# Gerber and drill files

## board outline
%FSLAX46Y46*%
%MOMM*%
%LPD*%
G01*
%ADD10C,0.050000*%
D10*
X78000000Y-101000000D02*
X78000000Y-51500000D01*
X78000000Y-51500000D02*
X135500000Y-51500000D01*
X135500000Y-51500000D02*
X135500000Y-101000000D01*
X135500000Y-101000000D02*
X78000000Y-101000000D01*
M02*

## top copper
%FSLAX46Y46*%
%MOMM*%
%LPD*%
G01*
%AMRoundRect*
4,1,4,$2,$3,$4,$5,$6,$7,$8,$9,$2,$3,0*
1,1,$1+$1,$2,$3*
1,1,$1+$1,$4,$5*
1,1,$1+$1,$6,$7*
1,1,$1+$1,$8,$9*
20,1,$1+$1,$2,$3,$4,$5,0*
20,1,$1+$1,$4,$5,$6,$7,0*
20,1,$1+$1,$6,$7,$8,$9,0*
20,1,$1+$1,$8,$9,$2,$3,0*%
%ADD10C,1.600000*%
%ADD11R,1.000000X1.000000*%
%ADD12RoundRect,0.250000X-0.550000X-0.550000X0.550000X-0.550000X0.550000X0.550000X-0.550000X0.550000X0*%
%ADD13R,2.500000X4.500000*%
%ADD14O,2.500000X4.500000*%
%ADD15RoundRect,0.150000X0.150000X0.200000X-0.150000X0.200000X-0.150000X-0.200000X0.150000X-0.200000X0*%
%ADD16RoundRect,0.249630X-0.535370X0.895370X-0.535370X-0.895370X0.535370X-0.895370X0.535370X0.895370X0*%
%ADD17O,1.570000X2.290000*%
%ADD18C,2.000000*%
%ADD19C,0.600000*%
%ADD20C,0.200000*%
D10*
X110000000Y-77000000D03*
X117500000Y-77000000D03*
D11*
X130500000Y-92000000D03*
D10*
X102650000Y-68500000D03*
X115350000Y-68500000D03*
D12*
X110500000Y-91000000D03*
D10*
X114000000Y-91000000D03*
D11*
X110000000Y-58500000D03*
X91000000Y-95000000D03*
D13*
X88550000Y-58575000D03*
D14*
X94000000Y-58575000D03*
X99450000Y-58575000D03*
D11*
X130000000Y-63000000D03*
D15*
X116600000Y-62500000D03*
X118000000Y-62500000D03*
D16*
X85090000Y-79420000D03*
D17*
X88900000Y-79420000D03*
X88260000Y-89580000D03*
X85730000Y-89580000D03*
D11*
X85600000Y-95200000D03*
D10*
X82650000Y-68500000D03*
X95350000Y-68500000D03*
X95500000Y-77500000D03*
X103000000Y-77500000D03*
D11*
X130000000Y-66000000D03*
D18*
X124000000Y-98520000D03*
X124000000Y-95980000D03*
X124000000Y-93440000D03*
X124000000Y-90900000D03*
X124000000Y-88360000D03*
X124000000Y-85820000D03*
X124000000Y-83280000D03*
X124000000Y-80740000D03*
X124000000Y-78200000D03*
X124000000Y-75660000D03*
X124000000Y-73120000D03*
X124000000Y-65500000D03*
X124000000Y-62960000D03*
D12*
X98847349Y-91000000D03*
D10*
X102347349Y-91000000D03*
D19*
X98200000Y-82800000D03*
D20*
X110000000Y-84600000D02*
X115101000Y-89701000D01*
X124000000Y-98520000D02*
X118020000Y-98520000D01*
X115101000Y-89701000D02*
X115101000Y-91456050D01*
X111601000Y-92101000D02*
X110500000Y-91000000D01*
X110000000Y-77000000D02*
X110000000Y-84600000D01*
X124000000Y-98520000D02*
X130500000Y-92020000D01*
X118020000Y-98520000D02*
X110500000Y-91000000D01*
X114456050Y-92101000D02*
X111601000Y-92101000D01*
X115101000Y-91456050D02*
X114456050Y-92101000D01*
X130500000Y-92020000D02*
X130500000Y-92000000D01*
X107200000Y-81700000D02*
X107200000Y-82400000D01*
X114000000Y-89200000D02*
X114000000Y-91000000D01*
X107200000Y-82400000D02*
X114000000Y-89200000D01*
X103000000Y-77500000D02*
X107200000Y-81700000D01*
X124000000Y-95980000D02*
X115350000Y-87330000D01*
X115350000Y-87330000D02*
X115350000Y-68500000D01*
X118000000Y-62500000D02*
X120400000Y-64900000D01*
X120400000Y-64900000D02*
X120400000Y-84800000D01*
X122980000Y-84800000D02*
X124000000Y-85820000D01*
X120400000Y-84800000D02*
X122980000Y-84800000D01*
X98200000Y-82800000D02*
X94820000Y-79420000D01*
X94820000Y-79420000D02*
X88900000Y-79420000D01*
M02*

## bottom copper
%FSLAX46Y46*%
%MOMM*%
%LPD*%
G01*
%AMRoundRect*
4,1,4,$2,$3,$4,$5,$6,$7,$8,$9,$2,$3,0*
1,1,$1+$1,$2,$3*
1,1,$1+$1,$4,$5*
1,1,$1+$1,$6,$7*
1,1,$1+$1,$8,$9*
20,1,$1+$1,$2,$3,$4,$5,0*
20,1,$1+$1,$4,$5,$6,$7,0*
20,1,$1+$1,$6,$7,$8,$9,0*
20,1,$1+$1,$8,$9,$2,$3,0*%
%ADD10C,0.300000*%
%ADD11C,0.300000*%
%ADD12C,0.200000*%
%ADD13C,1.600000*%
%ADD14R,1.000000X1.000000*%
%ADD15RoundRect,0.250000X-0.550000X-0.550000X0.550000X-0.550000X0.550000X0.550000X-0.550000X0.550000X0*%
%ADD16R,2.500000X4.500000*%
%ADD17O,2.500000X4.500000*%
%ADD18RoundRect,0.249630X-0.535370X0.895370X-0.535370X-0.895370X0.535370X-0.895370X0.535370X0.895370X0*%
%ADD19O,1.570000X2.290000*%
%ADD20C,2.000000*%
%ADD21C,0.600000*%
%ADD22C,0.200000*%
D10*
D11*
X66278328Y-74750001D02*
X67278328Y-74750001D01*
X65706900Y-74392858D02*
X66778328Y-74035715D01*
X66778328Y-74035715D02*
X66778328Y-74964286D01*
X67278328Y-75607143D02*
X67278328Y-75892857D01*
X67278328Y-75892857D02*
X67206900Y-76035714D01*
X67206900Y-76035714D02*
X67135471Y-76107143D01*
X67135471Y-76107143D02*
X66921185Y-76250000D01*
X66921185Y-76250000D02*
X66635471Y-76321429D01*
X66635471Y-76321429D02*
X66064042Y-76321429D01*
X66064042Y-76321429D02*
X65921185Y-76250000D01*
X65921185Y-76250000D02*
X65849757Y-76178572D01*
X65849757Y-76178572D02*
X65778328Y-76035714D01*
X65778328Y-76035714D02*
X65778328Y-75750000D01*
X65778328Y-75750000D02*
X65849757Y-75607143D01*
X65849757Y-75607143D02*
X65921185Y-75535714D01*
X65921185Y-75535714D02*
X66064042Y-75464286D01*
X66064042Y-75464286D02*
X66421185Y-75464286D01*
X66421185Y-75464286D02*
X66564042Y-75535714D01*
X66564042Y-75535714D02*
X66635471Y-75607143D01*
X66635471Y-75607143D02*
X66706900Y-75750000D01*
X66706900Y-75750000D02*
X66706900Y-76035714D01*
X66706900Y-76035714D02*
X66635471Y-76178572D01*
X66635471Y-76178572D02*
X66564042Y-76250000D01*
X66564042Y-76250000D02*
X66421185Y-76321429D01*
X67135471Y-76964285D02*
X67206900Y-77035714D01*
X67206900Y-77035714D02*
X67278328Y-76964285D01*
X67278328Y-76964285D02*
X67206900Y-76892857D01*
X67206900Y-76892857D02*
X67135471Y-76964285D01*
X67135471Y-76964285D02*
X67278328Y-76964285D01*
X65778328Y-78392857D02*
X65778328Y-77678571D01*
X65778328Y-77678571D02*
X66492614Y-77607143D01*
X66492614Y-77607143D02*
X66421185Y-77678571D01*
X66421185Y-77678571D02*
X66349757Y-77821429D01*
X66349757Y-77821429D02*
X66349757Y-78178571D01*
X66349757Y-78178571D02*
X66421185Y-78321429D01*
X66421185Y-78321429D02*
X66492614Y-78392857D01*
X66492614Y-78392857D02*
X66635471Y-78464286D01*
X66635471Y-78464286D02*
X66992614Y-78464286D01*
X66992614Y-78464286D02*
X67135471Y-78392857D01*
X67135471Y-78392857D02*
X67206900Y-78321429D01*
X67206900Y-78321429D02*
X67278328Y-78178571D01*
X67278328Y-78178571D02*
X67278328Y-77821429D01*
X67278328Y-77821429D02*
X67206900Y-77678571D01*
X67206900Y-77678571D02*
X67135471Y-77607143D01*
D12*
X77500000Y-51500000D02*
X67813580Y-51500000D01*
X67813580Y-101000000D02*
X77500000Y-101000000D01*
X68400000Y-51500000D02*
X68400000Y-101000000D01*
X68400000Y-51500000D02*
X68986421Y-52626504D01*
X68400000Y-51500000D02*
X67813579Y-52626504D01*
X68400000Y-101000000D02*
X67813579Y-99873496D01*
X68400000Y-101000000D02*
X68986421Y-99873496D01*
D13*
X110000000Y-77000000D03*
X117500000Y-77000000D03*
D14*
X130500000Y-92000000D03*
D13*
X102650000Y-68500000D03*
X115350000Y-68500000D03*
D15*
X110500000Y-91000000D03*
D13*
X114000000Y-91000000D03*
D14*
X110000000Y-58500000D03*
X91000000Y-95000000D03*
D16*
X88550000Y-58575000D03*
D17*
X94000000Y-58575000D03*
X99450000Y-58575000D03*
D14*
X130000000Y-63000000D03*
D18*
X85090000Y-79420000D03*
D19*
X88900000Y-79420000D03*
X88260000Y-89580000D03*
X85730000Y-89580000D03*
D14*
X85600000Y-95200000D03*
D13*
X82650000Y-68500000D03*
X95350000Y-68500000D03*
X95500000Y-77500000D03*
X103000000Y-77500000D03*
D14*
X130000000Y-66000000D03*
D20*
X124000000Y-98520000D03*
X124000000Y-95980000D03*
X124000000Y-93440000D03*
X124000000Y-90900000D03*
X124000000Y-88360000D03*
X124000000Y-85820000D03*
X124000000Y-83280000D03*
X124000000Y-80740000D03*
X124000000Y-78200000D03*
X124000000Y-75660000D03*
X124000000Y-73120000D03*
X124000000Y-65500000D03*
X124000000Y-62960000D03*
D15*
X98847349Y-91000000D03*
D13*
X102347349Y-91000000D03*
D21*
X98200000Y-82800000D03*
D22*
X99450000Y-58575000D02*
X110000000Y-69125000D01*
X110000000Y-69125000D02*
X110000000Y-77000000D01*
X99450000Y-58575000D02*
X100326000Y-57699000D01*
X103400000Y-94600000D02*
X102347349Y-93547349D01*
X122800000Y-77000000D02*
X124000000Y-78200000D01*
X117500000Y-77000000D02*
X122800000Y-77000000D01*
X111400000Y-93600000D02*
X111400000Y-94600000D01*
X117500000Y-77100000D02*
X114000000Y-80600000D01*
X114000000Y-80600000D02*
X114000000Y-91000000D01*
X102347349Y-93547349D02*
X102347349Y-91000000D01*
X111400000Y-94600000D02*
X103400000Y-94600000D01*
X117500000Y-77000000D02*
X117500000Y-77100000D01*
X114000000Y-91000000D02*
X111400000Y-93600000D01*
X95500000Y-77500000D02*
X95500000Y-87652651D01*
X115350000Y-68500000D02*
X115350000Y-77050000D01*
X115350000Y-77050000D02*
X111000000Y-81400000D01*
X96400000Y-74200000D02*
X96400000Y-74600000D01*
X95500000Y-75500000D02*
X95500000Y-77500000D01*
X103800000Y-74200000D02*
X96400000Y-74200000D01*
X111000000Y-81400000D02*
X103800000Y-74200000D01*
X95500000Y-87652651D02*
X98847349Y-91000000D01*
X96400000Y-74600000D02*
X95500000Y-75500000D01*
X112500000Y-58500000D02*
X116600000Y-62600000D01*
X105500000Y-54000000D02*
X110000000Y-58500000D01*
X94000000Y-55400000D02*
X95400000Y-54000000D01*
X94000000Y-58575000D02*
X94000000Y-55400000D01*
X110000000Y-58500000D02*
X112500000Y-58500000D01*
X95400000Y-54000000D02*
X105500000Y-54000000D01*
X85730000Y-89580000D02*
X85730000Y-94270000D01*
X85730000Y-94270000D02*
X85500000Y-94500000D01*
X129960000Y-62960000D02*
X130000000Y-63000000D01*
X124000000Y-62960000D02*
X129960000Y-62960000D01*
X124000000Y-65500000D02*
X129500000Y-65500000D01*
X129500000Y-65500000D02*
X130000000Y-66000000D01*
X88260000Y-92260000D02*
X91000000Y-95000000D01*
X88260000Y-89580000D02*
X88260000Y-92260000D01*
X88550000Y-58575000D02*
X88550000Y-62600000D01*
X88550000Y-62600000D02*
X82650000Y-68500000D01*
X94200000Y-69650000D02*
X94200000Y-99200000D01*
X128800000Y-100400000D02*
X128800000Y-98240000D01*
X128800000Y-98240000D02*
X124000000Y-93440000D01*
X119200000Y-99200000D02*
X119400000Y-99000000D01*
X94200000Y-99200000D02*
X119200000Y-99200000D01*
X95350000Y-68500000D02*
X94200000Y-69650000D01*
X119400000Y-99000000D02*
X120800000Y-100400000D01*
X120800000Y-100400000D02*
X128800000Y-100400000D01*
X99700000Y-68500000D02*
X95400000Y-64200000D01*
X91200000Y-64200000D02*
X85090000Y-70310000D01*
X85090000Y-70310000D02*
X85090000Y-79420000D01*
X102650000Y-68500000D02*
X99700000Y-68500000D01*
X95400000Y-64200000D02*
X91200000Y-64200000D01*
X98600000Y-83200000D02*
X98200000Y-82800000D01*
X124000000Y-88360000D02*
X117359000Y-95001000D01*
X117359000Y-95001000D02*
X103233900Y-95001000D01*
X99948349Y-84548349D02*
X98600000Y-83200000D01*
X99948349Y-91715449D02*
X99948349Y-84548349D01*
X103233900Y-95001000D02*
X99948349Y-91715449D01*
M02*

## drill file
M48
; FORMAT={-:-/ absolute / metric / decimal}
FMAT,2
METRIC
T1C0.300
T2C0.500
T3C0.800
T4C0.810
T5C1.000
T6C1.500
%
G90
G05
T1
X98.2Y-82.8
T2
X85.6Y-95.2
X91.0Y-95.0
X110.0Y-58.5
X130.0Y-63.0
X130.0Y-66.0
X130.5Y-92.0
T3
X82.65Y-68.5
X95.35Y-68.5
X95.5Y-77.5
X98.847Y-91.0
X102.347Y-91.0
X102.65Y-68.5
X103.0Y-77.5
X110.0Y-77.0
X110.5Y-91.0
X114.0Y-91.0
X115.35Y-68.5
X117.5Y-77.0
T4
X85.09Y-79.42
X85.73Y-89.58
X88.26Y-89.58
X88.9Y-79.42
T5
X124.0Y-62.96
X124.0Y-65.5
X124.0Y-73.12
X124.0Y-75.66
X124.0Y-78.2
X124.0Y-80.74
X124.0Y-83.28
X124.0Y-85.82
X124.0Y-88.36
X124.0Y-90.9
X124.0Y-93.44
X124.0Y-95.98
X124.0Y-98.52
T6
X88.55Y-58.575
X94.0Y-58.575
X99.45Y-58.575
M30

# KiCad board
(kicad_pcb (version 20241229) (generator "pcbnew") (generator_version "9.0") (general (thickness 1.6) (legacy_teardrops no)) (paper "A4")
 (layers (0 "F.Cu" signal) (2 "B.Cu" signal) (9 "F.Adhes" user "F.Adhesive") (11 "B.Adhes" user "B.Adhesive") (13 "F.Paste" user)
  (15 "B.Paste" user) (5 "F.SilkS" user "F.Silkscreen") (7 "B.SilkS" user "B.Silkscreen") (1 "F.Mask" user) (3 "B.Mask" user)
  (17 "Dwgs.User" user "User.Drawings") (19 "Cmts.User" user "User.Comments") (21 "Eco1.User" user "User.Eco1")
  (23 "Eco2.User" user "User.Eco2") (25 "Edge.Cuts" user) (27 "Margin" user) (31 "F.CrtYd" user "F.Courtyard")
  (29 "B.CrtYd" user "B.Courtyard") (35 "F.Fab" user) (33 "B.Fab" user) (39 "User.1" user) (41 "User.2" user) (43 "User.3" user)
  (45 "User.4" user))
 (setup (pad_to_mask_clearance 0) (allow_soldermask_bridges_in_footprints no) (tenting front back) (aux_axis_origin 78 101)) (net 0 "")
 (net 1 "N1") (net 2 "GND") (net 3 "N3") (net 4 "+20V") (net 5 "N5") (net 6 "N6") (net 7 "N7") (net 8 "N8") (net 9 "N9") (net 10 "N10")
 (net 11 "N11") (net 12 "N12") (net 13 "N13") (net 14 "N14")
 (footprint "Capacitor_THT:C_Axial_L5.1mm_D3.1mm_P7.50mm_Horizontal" (layer "F.Cu") (at 110 77)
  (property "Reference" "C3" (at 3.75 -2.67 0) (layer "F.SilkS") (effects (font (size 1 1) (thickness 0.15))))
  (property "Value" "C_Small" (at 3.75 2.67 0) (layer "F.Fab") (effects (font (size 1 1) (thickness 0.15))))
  (pad "1" thru_hole circle (at 0 0) (size 1.6 1.6) (drill 0.8) (layers "*.Cu" "*.Mask") (remove_unused_layers no) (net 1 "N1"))
  (pad "2" thru_hole circle (at 7.5 0) (size 1.6 1.6) (drill 0.8) (layers "*.Cu" "*.Mask") (remove_unused_layers no) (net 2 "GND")))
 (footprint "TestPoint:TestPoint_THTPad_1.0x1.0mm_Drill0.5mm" (layer "F.Cu") (at 130.5 92)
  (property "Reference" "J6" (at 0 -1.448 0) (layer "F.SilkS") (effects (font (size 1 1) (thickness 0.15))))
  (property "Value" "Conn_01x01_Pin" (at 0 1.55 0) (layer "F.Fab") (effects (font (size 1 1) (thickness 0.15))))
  (pad "1" thru_hole rect (at 0 0) (size 1 1) (drill 0.5) (layers "*.Cu" "*.Mask") (remove_unused_layers no) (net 1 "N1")))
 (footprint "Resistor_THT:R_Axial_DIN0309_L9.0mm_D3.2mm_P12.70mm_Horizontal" (layer "F.Cu") (at 102.65 68.5)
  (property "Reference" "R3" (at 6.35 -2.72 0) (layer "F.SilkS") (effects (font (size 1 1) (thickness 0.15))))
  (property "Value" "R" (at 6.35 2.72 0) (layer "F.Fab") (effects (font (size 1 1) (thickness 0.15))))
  (pad "1" thru_hole circle (at 0 0) (size 1.6 1.6) (drill 0.8) (layers "*.Cu" "*.Mask") (remove_unused_layers no) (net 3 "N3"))
  (pad "2" thru_hole circle (at 12.7 0) (size 1.6 1.6) (drill 0.8) (layers "*.Cu" "*.Mask") (remove_unused_layers no) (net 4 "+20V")))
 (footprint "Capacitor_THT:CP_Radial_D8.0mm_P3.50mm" (layer "F.Cu") (at 110.5 91)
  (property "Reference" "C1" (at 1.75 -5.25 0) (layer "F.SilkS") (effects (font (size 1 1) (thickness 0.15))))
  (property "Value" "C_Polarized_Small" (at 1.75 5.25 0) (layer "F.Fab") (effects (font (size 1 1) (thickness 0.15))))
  (pad "1" thru_hole roundrect (at 0 0) (size 1.6 1.6) (drill 0.8) (layers "*.Cu" "*.Mask") (remove_unused_layers no)
   (roundrect_rratio 0.15625) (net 1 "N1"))
  (pad "2" thru_hole circle (at 3.5 0) (size 1.6 1.6) (drill 0.8) (layers "*.Cu" "*.Mask") (remove_unused_layers no) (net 2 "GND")))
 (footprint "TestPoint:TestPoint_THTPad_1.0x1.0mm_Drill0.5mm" (layer "F.Cu") (at 110 58.5)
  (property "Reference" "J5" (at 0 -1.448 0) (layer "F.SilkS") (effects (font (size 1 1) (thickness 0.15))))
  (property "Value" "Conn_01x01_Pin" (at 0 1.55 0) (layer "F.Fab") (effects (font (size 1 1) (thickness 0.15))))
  (pad "1" thru_hole rect (at 0 0) (size 1 1) (drill 0.5) (layers "*.Cu" "*.Mask") (remove_unused_layers no) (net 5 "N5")))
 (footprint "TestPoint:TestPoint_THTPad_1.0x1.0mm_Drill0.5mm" (layer "F.Cu") (at 91 95)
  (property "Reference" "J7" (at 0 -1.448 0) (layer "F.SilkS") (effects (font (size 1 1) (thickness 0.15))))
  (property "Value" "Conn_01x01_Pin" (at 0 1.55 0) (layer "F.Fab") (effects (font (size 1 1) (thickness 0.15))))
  (pad "1" thru_hole rect (at 0 0) (size 1 1) (drill 0.5) (layers "*.Cu" "*.Mask") (remove_unused_layers no) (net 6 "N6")))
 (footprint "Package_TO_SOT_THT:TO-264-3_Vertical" (layer "F.Cu") (at 88.55 58.575)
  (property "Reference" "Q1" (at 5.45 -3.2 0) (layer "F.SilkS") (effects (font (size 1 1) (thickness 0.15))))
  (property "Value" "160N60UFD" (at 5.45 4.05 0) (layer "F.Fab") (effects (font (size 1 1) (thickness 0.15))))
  (pad "1" thru_hole rect (at 0 0) (size 2.5 4.5) (drill 1.5) (layers "*.Cu" "*.Mask") (remove_unused_layers no) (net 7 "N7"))
  (pad "2" thru_hole oval (at 5.45 0) (size 2.5 4.5) (drill 1.5) (layers "*.Cu" "*.Mask") (remove_unused_layers no) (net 5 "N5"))
  (pad "3" thru_hole oval (at 10.9 0) (size 2.5 4.5) (drill 1.5) (layers "*.Cu" "*.Mask") (remove_unused_layers no) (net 1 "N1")))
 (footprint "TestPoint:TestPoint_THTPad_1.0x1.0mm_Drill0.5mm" (layer "F.Cu") (at 130 63)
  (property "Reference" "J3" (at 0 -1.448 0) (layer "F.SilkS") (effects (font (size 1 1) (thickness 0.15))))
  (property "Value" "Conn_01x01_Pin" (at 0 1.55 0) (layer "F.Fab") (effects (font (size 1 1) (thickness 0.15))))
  (pad "1" thru_hole rect (at 0 0) (size 1 1) (drill 0.5) (layers "*.Cu" "*.Mask") (remove_unused_layers no) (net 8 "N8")))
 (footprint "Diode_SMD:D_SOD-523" (layer "F.Cu") (at 117.3 62.5)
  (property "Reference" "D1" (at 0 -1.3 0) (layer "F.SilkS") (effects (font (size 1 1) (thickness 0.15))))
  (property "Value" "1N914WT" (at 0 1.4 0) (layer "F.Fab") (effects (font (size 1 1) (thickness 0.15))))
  (pad "1" smd roundrect (at -0.7 0 180) (size 0.6 0.7) (layers "F.Cu" "F.Mask" "F.Paste") (roundrect_rratio 0.25) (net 5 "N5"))
  (pad "2" smd roundrect (at 0.7 0 180) (size 0.6 0.7) (layers "F.Cu" "F.Mask" "F.Paste") (roundrect_rratio 0.25) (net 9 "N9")))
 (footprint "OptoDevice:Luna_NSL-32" (layer "F.Cu") (at 85.09 79.42 -90)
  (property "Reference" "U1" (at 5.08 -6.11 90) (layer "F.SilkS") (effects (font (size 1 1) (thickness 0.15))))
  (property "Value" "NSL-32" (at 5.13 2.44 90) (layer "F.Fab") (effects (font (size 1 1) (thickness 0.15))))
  (pad "1" thru_hole roundrect (at 0 0 270) (size 2.29 1.57) (drill 0.81) (layers "*.Cu" "*.Mask") (remove_unused_layers no)
   (roundrect_rratio 0.159) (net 3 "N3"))
  (pad "2" thru_hole oval (at 0 -3.81 270) (size 2.29 1.57) (drill 0.81) (layers "*.Cu" "*.Mask") (remove_unused_layers no) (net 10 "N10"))
  (pad "3" thru_hole oval (at 10.16 -3.17 270) (size 2.29 1.57) (drill 0.81) (layers "*.Cu" "*.Mask") (remove_unused_layers no) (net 6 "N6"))
  (pad "4" thru_hole oval (at 10.16 -0.64 270) (size 2.29 1.57) (drill 0.81) (layers "*.Cu" "*.Mask") (remove_unused_layers no)
   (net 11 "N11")))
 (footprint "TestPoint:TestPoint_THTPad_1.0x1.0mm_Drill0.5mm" (layer "F.Cu") (at 85.6 95.2)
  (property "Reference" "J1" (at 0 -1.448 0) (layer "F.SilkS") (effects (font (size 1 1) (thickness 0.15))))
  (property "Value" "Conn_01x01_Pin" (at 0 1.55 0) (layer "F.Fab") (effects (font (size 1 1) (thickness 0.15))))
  (pad "1" thru_hole rect (at 0 0) (size 1 1) (drill 0.5) (layers "*.Cu" "*.Mask") (remove_unused_layers no) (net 11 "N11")))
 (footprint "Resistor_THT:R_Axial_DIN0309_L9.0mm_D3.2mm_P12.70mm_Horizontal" (layer "F.Cu") (at 82.65 68.5)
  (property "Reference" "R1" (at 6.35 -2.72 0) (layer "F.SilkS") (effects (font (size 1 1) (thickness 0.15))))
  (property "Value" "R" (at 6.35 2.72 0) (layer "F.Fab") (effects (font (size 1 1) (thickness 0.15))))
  (pad "1" thru_hole circle (at 0 0) (size 1.6 1.6) (drill 0.8) (layers "*.Cu" "*.Mask") (remove_unused_layers no) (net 7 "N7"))
  (pad "2" thru_hole circle (at 12.7 0) (size 1.6 1.6) (drill 0.8) (layers "*.Cu" "*.Mask") (remove_unused_layers no) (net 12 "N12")))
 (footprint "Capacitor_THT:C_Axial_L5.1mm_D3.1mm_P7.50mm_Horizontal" (layer "F.Cu") (at 95.5 77.5)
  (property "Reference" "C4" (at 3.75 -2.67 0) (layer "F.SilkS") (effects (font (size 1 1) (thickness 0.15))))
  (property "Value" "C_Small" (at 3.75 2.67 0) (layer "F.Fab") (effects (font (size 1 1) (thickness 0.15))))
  (pad "1" thru_hole circle (at 0 0) (size 1.6 1.6) (drill 0.8) (layers "*.Cu" "*.Mask") (remove_unused_layers no) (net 4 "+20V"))
  (pad "2" thru_hole circle (at 7.5 0) (size 1.6 1.6) (drill 0.8) (layers "*.Cu" "*.Mask") (remove_unused_layers no) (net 2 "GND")))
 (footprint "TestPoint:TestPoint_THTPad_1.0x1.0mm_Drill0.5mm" (layer "F.Cu") (at 130 66)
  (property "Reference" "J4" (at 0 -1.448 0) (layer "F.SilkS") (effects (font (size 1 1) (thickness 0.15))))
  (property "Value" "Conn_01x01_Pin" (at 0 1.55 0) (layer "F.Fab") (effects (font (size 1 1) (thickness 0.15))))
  (pad "1" thru_hole rect (at 0 0) (size 1 1) (drill 0.5) (layers "*.Cu" "*.Mask") (remove_unused_layers no) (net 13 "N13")))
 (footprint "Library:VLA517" (layer "F.Cu") (at 124 80.74 90)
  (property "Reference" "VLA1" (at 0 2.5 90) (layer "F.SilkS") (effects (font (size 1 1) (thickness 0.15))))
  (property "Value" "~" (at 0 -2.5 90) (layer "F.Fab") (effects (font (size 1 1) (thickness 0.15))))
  (pad "1" thru_hole circle (at -17.78 0 90) (size 2 2) (drill 1) (layers "*.Cu" "*.Mask") (remove_unused_layers no) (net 1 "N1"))
  (pad "2" thru_hole circle (at -15.24 0 90) (size 2 2) (drill 1) (layers "*.Cu" "*.Mask") (remove_unused_layers no) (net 4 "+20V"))
  (pad "3" thru_hole circle (at -12.7 0 90) (size 2 2) (drill 1) (layers "*.Cu" "*.Mask") (remove_unused_layers no) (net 12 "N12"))
  (pad "4" thru_hole circle (at -10.16 0 90) (size 2 2) (drill 1) (layers "*.Cu" "*.Mask") (remove_unused_layers no) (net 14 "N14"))
  (pad "5" thru_hole circle (at -7.62 0 90) (size 2 2) (drill 1) (layers "*.Cu" "*.Mask") (remove_unused_layers no) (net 10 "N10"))
  (pad "6" thru_hole circle (at -5.08 0 90) (size 2 2) (drill 1) (layers "*.Cu" "*.Mask") (remove_unused_layers no) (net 9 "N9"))
  (pad "7" thru_hole circle (at -2.54 0 90) (size 2 2) (drill 1) (layers "*.Cu" "*.Mask") (remove_unused_layers no))
  (pad "8" thru_hole circle (at 0 0 90) (size 2 2) (drill 1) (layers "*.Cu" "*.Mask") (remove_unused_layers no))
  (pad "9" thru_hole circle (at 2.54 0 90) (size 2 2) (drill 1) (layers "*.Cu" "*.Mask") (remove_unused_layers no) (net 2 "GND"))
  (pad "10" thru_hole circle (at 5.08 0 90) (size 2 2) (drill 1) (layers "*.Cu" "*.Mask") (remove_unused_layers no))
  (pad "11" thru_hole circle (at 7.62 0 90) (size 2 2) (drill 1) (layers "*.Cu" "*.Mask") (remove_unused_layers no))
  (pad "14" thru_hole circle (at 15.24 0 90) (size 2 2) (drill 1) (layers "*.Cu" "*.Mask") (remove_unused_layers no) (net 13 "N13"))
  (pad "15" thru_hole circle (at 17.78 0 90) (size 2 2) (drill 1) (layers "*.Cu" "*.Mask") (remove_unused_layers no) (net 8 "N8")))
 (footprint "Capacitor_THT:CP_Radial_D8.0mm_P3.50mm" (layer "F.Cu") (at 98.847349 91)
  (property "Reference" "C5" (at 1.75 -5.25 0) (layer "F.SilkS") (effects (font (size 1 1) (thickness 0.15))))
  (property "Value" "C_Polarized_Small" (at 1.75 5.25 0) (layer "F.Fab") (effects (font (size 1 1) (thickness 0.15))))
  (pad "1" thru_hole roundrect (at 0 0) (size 1.6 1.6) (drill 0.8) (layers "*.Cu" "*.Mask") (remove_unused_layers no)
   (roundrect_rratio 0.15625) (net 4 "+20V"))
  (pad "2" thru_hole circle (at 3.5 0) (size 1.6 1.6) (drill 0.8) (layers "*.Cu" "*.Mask") (remove_unused_layers no) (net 2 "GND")))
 (gr_line (start 78 101) (end 78 51.5) (stroke (width 0.05) (type default)) (layer "Edge.Cuts"))
 (gr_line (start 78 51.5) (end 135.5 51.5) (stroke (width 0.05) (type default)) (layer "Edge.Cuts"))
 (gr_line (start 135.5 51.5) (end 135.5 101) (stroke (width 0.05) (type default)) (layer "Edge.Cuts"))
 (gr_line (start 135.5 101) (end 78 101) (stroke (width 0.05) (type default)) (layer "Edge.Cuts"))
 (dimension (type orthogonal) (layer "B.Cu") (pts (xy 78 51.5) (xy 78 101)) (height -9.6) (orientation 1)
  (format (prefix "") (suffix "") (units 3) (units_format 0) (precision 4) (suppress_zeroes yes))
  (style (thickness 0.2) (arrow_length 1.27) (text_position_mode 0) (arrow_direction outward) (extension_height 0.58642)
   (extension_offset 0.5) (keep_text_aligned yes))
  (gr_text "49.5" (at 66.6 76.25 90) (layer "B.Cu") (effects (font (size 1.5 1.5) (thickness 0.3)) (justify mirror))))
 (segment (start 110 84.6) (end 115.101 89.701) (width 0.2) (layer "F.Cu") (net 1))
 (segment (start 124 98.52) (end 118.02 98.52) (width 0.2) (layer "F.Cu") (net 1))
 (segment (start 115.101 89.701) (end 115.101 91.45605) (width 0.2) (layer "F.Cu") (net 1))
 (segment (start 111.601 92.101) (end 110.5 91) (width 0.2) (layer "F.Cu") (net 1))
 (segment (start 110 77) (end 110 84.6) (width 0.2) (layer "F.Cu") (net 1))
 (segment (start 124 98.52) (end 130.5 92.02) (width 0.2) (layer "F.Cu") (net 1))
 (segment (start 118.02 98.52) (end 110.5 91) (width 0.2) (layer "F.Cu") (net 1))
 (segment (start 114.45605 92.101) (end 111.601 92.101) (width 0.2) (layer "F.Cu") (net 1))
 (segment (start 115.101 91.45605) (end 114.45605 92.101) (width 0.2) (layer "F.Cu") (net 1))
 (segment (start 130.5 92.02) (end 130.5 92) (width 0.2) (layer "F.Cu") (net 1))
 (segment (start 99.45 58.575) (end 110 69.125) (width 0.2) (layer "B.Cu") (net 1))
 (segment (start 110 69.125) (end 110 77) (width 0.2) (layer "B.Cu") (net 1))
 (segment (start 99.45 58.575) (end 100.326 57.699) (width 0.2) (layer "B.Cu") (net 1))
 (segment (start 107.2 81.7) (end 107.2 82.4) (width 0.2) (layer "F.Cu") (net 2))
 (segment (start 114 89.2) (end 114 91) (width 0.2) (layer "F.Cu") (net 2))
 (segment (start 107.2 82.4) (end 114 89.2) (width 0.2) (layer "F.Cu") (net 2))
 (segment (start 103 77.5) (end 107.2 81.7) (width 0.2) (layer "F.Cu") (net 2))
 (segment (start 103.4 94.6) (end 102.347349 93.547349) (width 0.2) (layer "B.Cu") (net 2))
 (segment (start 122.8 77) (end 124 78.2) (width 0.2) (layer "B.Cu") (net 2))
 (segment (start 117.5 77) (end 122.8 77) (width 0.2) (layer "B.Cu") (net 2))
 (segment (start 111.4 93.6) (end 111.4 94.6) (width 0.2) (layer "B.Cu") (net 2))
 (segment (start 117.5 77.1) (end 114 80.6) (width 0.2) (layer "B.Cu") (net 2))
 (segment (start 114 80.6) (end 114 91) (width 0.2) (layer "B.Cu") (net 2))
 (segment (start 102.347349 93.547349) (end 102.347349 91) (width 0.2) (layer "B.Cu") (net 2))
 (segment (start 111.4 94.6) (end 103.4 94.6) (width 0.2) (layer "B.Cu") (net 2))
 (segment (start 117.5 77) (end 117.5 77.1) (width 0.2) (layer "B.Cu") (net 2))
 (segment (start 114 91) (end 111.4 93.6) (width 0.2) (layer "B.Cu") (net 2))
 (segment (start 124 95.98) (end 115.35 87.33) (width 0.2) (layer "F.Cu") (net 4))
 (segment (start 115.35 87.33) (end 115.35 68.5) (width 0.2) (layer "F.Cu") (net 4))
 (segment (start 95.5 77.5) (end 95.5 87.652651) (width 0.2) (layer "B.Cu") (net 4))
 (segment (start 115.35 68.5) (end 115.35 77.05) (width 0.2) (layer "B.Cu") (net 4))
 (segment (start 115.35 77.05) (end 111 81.4) (width 0.2) (layer "B.Cu") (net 4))
 (segment (start 96.4 74.2) (end 96.4 74.6) (width 0.2) (layer "B.Cu") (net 4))
 (segment (start 95.5 75.5) (end 95.5 77.5) (width 0.2) (layer "B.Cu") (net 4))
 (segment (start 103.8 74.2) (end 96.4 74.2) (width 0.2) (layer "B.Cu") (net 4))
 (segment (start 111 81.4) (end 103.8 74.2) (width 0.2) (layer "B.Cu") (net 4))
 (segment (start 95.5 87.652651) (end 98.847349 91) (width 0.2) (layer "B.Cu") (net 4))
 (segment (start 96.4 74.6) (end 95.5 75.5) (width 0.2) (layer "B.Cu") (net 4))
 (segment (start 112.5 58.5) (end 116.6 62.6) (width 0.2) (layer "B.Cu") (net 5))
 (segment (start 105.5 54) (end 110 58.5) (width 0.2) (layer "B.Cu") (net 5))
 (segment (start 94 55.4) (end 95.4 54) (width 0.2) (layer "B.Cu") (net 5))
 (segment (start 94 58.575) (end 94 55.4) (width 0.2) (layer "B.Cu") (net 5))
 (segment (start 110 58.5) (end 112.5 58.5) (width 0.2) (layer "B.Cu") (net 5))
 (segment (start 95.4 54) (end 105.5 54) (width 0.2) (layer "B.Cu") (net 5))
 (segment (start 118 62.5) (end 120.4 64.9) (width 0.2) (layer "F.Cu") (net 9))
 (segment (start 120.4 64.9) (end 120.4 84.8) (width 0.2) (layer "F.Cu") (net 9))
 (segment (start 122.98 84.8) (end 124 85.82) (width 0.2) (layer "F.Cu") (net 9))
 (segment (start 120.4 84.8) (end 122.98 84.8) (width 0.2) (layer "F.Cu") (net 9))
 (segment (start 85.73 89.58) (end 85.73 94.27) (width 0.2) (layer "B.Cu") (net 11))
 (segment (start 85.73 94.27) (end 85.5 94.5) (width 0.2) (layer "B.Cu") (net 11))
 (segment (start 129.96 62.96) (end 130 63) (width 0.2) (layer "B.Cu") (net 8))
 (segment (start 124 62.96) (end 129.96 62.96) (width 0.2) (layer "B.Cu") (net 8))
 (segment (start 124 65.5) (end 129.5 65.5) (width 0.2) (layer "B.Cu") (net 13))
 (segment (start 129.5 65.5) (end 130 66) (width 0.2) (layer "B.Cu") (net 13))
 (segment (start 88.26 92.26) (end 91 95) (width 0.2) (layer "B.Cu") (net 6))
 (segment (start 88.26 89.58) (end 88.26 92.26) (width 0.2) (layer "B.Cu") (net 6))
 (segment (start 88.55 58.575) (end 88.55 62.6) (width 0.2) (layer "B.Cu") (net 7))
 (segment (start 88.55 62.6) (end 82.65 68.5) (width 0.2) (layer "B.Cu") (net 7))
 (segment (start 94.2 69.65) (end 94.2 99.2) (width 0.2) (layer "B.Cu") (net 12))
 (segment (start 128.8 100.4) (end 128.8 98.24) (width 0.2) (layer "B.Cu") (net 12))
 (segment (start 128.8 98.24) (end 124 93.44) (width 0.2) (layer "B.Cu") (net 12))
 (segment (start 119.2 99.2) (end 119.4 99) (width 0.2) (layer "B.Cu") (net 12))
 (segment (start 94.2 99.2) (end 119.2 99.2) (width 0.2) (layer "B.Cu") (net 12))
 (segment (start 95.35 68.5) (end 94.2 69.65) (width 0.2) (layer "B.Cu") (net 12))
 (segment (start 119.4 99) (end 120.8 100.4) (width 0.2) (layer "B.Cu") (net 12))
 (segment (start 120.8 100.4) (end 128.8 100.4) (width 0.2) (layer "B.Cu") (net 12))
 (segment (start 99.7 68.5) (end 95.4 64.2) (width 0.2) (layer "B.Cu") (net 3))
 (segment (start 91.2 64.2) (end 85.09 70.31) (width 0.2) (layer "B.Cu") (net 3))
 (segment (start 85.09 70.31) (end 85.09 79.42) (width 0.2) (layer "B.Cu") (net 3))
 (segment (start 102.65 68.5) (end 99.7 68.5) (width 0.2) (layer "B.Cu") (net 3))
 (segment (start 95.4 64.2) (end 91.2 64.2) (width 0.2) (layer "B.Cu") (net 3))
 (segment (start 98.2 82.8) (end 94.82 79.42) (width 0.2) (layer "F.Cu") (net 10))
 (segment (start 94.82 79.42) (end 88.9 79.42) (width 0.2) (layer "F.Cu") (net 10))
 (via (at 98.2 82.8) (size 0.6) (drill 0.3) (layers "F.Cu" "B.Cu") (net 10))
 (segment (start 98.6 83.2) (end 98.2 82.8) (width 0.2) (layer "B.Cu") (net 10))
 (segment (start 124 88.36) (end 117.359 95.001) (width 0.2) (layer "B.Cu") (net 10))
 (segment (start 117.359 95.001) (end 103.2339 95.001) (width 0.2) (layer "B.Cu") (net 10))
 (segment (start 99.948349 84.548349) (end 98.6 83.2) (width 0.2) (layer "B.Cu") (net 10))
 (segment (start 99.948349 91.715449) (end 99.948349 84.548349) (width 0.2) (layer "B.Cu") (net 10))
 (segment (start 103.2339 95.001) (end 99.948349 91.715449) (width 0.2) (layer "B.Cu") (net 10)))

